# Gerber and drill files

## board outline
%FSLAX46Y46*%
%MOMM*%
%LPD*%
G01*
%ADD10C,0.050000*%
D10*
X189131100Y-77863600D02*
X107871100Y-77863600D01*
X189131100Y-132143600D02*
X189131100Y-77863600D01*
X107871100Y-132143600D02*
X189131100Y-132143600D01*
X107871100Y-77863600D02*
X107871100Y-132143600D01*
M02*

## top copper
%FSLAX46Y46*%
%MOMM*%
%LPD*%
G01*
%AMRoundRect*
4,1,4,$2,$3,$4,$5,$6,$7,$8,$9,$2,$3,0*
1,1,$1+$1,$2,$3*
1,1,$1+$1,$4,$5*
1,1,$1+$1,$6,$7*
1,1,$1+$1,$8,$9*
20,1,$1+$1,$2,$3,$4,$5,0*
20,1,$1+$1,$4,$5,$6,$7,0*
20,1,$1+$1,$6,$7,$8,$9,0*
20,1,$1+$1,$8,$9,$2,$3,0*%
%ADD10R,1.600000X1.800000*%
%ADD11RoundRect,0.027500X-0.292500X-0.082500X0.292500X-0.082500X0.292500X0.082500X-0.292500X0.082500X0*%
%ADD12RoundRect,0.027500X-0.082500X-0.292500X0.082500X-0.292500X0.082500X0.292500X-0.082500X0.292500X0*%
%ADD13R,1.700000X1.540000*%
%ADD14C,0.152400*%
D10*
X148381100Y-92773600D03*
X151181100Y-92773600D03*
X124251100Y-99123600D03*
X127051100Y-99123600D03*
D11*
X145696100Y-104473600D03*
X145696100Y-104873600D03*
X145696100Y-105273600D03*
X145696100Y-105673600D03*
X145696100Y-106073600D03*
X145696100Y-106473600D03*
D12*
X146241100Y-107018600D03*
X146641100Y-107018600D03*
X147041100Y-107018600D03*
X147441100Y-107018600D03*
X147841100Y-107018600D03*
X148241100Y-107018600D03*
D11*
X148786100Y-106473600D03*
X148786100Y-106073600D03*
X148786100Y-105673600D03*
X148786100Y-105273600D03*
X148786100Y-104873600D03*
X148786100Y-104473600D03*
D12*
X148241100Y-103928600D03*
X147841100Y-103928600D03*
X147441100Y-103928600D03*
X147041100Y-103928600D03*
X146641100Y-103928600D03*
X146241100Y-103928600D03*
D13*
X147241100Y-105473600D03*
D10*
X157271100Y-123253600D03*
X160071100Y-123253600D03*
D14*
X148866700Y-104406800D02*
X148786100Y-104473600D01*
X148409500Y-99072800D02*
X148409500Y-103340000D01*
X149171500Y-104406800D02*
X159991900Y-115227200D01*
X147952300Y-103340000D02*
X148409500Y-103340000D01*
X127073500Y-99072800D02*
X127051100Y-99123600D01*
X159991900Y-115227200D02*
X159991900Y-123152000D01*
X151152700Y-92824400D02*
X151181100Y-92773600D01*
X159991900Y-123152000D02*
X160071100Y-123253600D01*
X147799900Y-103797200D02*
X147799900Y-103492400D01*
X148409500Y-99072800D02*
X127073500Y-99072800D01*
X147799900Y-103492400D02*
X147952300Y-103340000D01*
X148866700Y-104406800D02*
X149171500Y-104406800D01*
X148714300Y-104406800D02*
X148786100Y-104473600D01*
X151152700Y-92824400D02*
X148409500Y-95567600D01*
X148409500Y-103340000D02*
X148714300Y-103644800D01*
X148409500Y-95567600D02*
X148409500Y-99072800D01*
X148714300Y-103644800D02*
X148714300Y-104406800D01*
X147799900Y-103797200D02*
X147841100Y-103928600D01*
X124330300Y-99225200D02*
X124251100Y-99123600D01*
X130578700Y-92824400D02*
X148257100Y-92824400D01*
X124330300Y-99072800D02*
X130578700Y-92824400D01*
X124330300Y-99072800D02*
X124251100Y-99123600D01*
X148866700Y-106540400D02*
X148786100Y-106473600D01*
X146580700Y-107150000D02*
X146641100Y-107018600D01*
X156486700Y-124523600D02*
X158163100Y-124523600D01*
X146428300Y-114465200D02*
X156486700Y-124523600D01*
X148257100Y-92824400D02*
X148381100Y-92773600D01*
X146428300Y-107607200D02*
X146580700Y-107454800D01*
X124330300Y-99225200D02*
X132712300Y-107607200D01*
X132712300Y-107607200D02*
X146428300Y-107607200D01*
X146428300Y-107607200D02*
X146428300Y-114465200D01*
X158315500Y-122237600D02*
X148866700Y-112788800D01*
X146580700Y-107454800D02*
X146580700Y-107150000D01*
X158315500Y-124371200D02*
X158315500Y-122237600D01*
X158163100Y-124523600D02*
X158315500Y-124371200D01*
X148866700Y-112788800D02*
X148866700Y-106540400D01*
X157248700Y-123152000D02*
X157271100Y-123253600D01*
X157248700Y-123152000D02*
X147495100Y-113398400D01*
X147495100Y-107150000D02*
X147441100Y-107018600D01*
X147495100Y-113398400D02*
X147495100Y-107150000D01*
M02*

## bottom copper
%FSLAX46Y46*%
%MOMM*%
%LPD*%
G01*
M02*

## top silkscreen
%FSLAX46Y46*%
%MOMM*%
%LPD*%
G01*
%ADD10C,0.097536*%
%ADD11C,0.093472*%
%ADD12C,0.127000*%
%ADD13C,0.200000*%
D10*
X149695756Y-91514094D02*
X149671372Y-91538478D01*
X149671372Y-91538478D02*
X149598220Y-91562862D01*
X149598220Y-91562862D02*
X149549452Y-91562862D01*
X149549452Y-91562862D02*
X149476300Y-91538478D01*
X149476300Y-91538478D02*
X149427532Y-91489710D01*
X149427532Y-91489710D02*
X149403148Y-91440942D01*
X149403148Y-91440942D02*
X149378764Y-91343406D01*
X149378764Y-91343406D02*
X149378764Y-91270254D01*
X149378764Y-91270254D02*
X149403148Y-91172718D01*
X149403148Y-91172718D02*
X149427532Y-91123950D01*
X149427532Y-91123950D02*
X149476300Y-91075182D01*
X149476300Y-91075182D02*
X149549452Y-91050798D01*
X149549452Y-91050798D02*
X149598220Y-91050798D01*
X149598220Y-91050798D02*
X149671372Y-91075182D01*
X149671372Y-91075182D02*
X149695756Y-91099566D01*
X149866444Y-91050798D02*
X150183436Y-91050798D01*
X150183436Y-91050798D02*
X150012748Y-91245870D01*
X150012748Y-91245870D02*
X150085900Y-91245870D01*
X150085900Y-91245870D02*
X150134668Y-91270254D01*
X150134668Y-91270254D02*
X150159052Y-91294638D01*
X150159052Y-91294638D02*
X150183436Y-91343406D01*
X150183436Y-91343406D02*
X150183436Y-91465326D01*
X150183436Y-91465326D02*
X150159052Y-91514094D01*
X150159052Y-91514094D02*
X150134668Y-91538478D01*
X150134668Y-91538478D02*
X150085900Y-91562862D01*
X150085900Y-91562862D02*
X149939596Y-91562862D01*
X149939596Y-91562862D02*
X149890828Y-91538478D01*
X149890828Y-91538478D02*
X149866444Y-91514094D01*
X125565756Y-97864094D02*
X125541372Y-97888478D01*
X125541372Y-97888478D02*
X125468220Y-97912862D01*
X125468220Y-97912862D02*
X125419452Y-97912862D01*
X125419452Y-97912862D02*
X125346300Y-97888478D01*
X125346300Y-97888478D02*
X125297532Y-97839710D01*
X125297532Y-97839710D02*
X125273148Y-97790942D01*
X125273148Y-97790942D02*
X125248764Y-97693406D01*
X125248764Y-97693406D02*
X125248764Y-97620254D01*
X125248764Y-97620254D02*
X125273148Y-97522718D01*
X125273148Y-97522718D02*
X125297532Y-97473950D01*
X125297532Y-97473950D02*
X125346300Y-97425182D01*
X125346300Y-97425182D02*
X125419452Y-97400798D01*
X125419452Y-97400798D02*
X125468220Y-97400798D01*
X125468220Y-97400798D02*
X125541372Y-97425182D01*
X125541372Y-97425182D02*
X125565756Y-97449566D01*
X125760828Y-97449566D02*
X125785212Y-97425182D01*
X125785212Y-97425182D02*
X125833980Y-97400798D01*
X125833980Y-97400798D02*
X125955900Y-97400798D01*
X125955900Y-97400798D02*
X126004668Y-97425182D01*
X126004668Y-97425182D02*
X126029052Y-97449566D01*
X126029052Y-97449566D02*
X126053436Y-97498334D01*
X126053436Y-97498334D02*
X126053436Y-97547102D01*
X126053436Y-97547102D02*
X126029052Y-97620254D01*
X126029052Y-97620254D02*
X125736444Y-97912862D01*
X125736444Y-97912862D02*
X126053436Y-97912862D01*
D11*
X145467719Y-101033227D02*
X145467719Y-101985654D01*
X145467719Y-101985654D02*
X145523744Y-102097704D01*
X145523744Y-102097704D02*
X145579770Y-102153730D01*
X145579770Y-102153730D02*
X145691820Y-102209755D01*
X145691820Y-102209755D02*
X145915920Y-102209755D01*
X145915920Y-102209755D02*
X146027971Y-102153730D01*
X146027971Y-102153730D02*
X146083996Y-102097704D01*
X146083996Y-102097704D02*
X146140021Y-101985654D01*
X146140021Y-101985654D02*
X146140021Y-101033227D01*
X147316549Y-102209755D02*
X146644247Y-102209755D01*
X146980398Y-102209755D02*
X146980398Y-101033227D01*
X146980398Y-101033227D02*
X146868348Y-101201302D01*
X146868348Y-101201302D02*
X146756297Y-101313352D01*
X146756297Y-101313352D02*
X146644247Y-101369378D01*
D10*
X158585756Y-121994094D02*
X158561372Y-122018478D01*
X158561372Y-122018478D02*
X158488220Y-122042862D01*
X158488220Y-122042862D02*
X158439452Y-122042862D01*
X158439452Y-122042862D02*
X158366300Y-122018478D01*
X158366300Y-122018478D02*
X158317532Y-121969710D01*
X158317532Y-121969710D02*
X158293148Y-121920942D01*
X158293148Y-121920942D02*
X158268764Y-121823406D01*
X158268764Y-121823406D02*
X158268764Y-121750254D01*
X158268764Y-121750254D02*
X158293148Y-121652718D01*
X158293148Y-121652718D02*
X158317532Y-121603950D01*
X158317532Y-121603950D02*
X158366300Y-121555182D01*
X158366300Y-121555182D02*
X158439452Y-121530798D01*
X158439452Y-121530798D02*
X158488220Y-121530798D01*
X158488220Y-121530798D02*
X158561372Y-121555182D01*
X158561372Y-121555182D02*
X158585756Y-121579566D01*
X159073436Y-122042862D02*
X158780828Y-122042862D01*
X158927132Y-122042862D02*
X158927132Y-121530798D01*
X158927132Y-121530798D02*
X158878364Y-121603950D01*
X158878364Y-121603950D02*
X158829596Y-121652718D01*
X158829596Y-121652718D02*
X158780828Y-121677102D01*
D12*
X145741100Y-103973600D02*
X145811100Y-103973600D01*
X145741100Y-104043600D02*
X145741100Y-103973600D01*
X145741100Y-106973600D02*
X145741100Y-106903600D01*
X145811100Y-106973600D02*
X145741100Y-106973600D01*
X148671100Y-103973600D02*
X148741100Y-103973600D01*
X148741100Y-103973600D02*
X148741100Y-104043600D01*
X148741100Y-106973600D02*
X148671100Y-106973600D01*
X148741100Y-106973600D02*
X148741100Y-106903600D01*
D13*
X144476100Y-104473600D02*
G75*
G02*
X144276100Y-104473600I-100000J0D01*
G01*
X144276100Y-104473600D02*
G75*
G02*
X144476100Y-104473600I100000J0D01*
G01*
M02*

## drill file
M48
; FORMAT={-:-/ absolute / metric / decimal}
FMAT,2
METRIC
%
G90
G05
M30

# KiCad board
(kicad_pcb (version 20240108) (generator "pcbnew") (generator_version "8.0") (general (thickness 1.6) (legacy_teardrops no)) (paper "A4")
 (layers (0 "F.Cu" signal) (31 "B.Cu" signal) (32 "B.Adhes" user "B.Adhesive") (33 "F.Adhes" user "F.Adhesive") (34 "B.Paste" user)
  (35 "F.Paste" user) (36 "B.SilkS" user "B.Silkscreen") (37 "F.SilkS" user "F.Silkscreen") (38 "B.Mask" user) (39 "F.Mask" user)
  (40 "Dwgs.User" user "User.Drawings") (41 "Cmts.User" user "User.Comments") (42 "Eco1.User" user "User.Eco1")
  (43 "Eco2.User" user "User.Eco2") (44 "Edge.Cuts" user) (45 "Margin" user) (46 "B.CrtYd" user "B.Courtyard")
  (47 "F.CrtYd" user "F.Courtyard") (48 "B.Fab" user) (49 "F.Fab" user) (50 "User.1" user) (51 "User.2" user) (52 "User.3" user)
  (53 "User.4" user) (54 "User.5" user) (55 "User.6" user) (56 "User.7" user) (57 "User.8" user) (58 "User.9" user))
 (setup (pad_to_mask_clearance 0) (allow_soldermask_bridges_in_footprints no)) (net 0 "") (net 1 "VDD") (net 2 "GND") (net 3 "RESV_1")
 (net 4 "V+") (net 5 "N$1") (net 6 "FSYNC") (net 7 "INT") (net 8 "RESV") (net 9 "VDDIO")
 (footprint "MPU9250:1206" (layer "F.Cu") (at 149.7811 92.7736)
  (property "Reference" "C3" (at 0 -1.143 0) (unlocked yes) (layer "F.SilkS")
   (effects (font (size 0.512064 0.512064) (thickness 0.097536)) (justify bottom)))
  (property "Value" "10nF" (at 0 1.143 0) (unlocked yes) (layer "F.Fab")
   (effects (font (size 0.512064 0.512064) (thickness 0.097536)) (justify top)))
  (pad "1" smd rect (at -1.4 0) (size 1.6 1.8) (layers "F.Cu" "F.Paste" "F.Mask") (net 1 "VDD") (solder_mask_margin 0.1016)
   (thermal_bridge_angle 0))
  (pad "2" smd rect (at 1.4 0) (size 1.6 1.8) (layers "F.Cu" "F.Paste" "F.Mask") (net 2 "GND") (solder_mask_margin 0.1016)
   (thermal_bridge_angle 0)))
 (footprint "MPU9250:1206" (layer "F.Cu") (at 125.6511 99.1236)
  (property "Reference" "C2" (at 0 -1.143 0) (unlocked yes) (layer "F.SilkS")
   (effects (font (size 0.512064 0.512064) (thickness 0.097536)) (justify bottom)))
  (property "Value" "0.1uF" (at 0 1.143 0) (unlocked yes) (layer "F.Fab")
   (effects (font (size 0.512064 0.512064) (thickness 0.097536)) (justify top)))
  (pad "1" smd rect (at -1.4 0) (size 1.6 1.8) (layers "F.Cu" "F.Paste" "F.Mask") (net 1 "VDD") (solder_mask_margin 0.1016)
   (thermal_bridge_angle 0))
  (pad "2" smd rect (at 1.4 0) (size 1.6 1.8) (layers "F.Cu" "F.Paste" "F.Mask") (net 2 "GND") (solder_mask_margin 0.1016)
   (thermal_bridge_angle 0)))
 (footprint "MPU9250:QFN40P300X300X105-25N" (layer "F.Cu") (at 147.2411 105.4736)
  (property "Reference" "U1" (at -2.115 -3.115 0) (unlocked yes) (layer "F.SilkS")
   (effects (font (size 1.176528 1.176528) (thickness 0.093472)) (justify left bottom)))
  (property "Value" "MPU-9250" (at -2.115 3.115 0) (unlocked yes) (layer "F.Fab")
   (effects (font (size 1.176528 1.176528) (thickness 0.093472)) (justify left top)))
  (fp_line (start -1.5 -1.5) (end -1.43 -1.5) (stroke (width 0.127) (type solid)) (layer "F.SilkS"))
  (fp_line (start -1.5 -1.43) (end -1.5 -1.5) (stroke (width 0.127) (type solid)) (layer "F.SilkS"))
  (fp_line (start -1.5 1.5) (end -1.5 1.43) (stroke (width 0.127) (type solid)) (layer "F.SilkS"))
  (fp_line (start -1.43 1.5) (end -1.5 1.5) (stroke (width 0.127) (type solid)) (layer "F.SilkS"))
  (fp_line (start 1.43 -1.5) (end 1.5 -1.5) (stroke (width 0.127) (type solid)) (layer "F.SilkS"))
  (fp_line (start 1.5 -1.5) (end 1.5 -1.43) (stroke (width 0.127) (type solid)) (layer "F.SilkS"))
  (fp_line (start 1.5 1.5) (end 1.43 1.5) (stroke (width 0.127) (type solid)) (layer "F.SilkS"))
  (fp_line (start 1.5 1.5) (end 1.5 1.43) (stroke (width 0.127) (type solid)) (layer "F.SilkS"))
  (fp_circle (center -2.865 -1) (end -2.765 -1) (stroke (width 0.2) (type solid)) (fill none) (layer "F.SilkS"))
  (pad "1" smd roundrect (at -1.545 -1) (size 0.64 0.22) (layers "F.Cu" "F.Paste" "F.Mask") (roundrect_rratio 0.125) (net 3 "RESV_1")
   (solder_mask_margin 0.1016) (thermal_bridge_angle 0))
  (pad "2" smd roundrect (at -1.545 -0.6) (size 0.64 0.22) (layers "F.Cu" "F.Paste" "F.Mask") (roundrect_rratio 0.125)
   (solder_mask_margin 0.1016) (thermal_bridge_angle 0))
  (pad "3" smd roundrect (at -1.545 -0.2) (size 0.64 0.22) (layers "F.Cu" "F.Paste" "F.Mask") (roundrect_rratio 0.125)
   (solder_mask_margin 0.1016) (thermal_bridge_angle 0))
  (pad "4" smd roundrect (at -1.545 0.2) (size 0.64 0.22) (layers "F.Cu" "F.Paste" "F.Mask") (roundrect_rratio 0.125)
   (solder_mask_margin 0.1016) (thermal_bridge_angle 0))
  (pad "5" smd roundrect (at -1.545 0.6) (size 0.64 0.22) (layers "F.Cu" "F.Paste" "F.Mask") (roundrect_rratio 0.125)
   (solder_mask_margin 0.1016) (thermal_bridge_angle 0))
  (pad "6" smd roundrect (at -1.545 1) (size 0.64 0.22) (layers "F.Cu" "F.Paste" "F.Mask") (roundrect_rratio 0.125)
   (solder_mask_margin 0.1016) (thermal_bridge_angle 0))
  (pad "7" smd roundrect (at -1 1.545) (size 0.22 0.64) (layers "F.Cu" "F.Paste" "F.Mask") (roundrect_rratio 0.125)
   (solder_mask_margin 0.1016) (thermal_bridge_angle 0))
  (pad "8" smd roundrect (at -0.6 1.545) (size 0.22 0.64) (layers "F.Cu" "F.Paste" "F.Mask") (roundrect_rratio 0.125) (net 1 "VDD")
   (solder_mask_margin 0.1016) (thermal_bridge_angle 0))
  (pad "9" smd roundrect (at -0.2 1.545) (size 0.22 0.64) (layers "F.Cu" "F.Paste" "F.Mask") (roundrect_rratio 0.125) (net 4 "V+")
   (solder_mask_margin 0.1016) (thermal_bridge_angle 0))
  (pad "10" smd roundrect (at 0.2 1.545) (size 0.22 0.64) (layers "F.Cu" "F.Paste" "F.Mask") (roundrect_rratio 0.125) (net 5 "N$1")
   (solder_mask_margin 0.1016) (thermal_bridge_angle 0))
  (pad "11" smd roundrect (at 0.6 1.545) (size 0.22 0.64) (layers "F.Cu" "F.Paste" "F.Mask") (roundrect_rratio 0.125) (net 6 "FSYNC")
   (solder_mask_margin 0.1016) (thermal_bridge_angle 0))
  (pad "12" smd roundrect (at 1 1.545) (size 0.22 0.64) (layers "F.Cu" "F.Paste" "F.Mask") (roundrect_rratio 0.125) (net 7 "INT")
   (solder_mask_margin 0.1016) (thermal_bridge_angle 0))
  (pad "13" smd roundrect (at 1.545 1) (size 0.64 0.22) (layers "F.Cu" "F.Paste" "F.Mask") (roundrect_rratio 0.125) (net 1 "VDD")
   (solder_mask_margin 0.1016) (thermal_bridge_angle 0))
  (pad "14" smd roundrect (at 1.545 0.6) (size 0.64 0.22) (layers "F.Cu" "F.Paste" "F.Mask") (roundrect_rratio 0.125)
   (solder_mask_margin 0.1016) (thermal_bridge_angle 0))
  (pad "15" smd roundrect (at 1.545 0.2) (size 0.64 0.22) (layers "F.Cu" "F.Paste" "F.Mask") (roundrect_rratio 0.125)
   (solder_mask_margin 0.1016) (thermal_bridge_angle 0))
  (pad "16" smd roundrect (at 1.545 -0.2) (size 0.64 0.22) (layers "F.Cu" "F.Paste" "F.Mask") (roundrect_rratio 0.125)
   (solder_mask_margin 0.1016) (thermal_bridge_angle 0))
  (pad "17" smd roundrect (at 1.545 -0.6) (size 0.64 0.22) (layers "F.Cu" "F.Paste" "F.Mask") (roundrect_rratio 0.125)
   (solder_mask_margin 0.1016) (thermal_bridge_angle 0))
  (pad "18" smd roundrect (at 1.545 -1) (size 0.64 0.22) (layers "F.Cu" "F.Paste" "F.Mask") (roundrect_rratio 0.125) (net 2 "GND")
   (solder_mask_margin 0.1016) (thermal_bridge_angle 0))
  (pad "19" smd roundrect (at 1 -1.545) (size 0.22 0.64) (layers "F.Cu" "F.Paste" "F.Mask") (roundrect_rratio 0.125) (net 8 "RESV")
   (solder_mask_margin 0.1016) (thermal_bridge_angle 0))
  (pad "20" smd roundrect (at 0.6 -1.545) (size 0.22 0.64) (layers "F.Cu" "F.Paste" "F.Mask") (roundrect_rratio 0.125) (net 2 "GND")
   (solder_mask_margin 0.1016) (thermal_bridge_angle 0))
  (pad "21" smd roundrect (at 0.2 -1.545) (size 0.22 0.64) (layers "F.Cu" "F.Paste" "F.Mask") (roundrect_rratio 0.125)
   (solder_mask_margin 0.1016) (thermal_bridge_angle 0))
  (pad "22" smd roundrect (at -0.2 -1.545) (size 0.22 0.64) (layers "F.Cu" "F.Paste" "F.Mask") (roundrect_rratio 0.125) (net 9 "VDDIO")
   (solder_mask_margin 0.1016) (thermal_bridge_angle 0))
  (pad "23" smd roundrect (at -0.6 -1.545) (size 0.22 0.64) (layers "F.Cu" "F.Paste" "F.Mask") (roundrect_rratio 0.125)
   (solder_mask_margin 0.1016) (thermal_bridge_angle 0))
  (pad "24" smd roundrect (at -1 -1.545) (size 0.22 0.64) (layers "F.Cu" "F.Paste" "F.Mask") (roundrect_rratio 0.125)
   (solder_mask_margin 0.1016) (thermal_bridge_angle 0))
  (pad "25" smd rect (at 0 0) (size 1.7 1.54) (layers "F.Cu" "F.Mask") (solder_mask_margin 0.1016) (thermal_bridge_angle 0)))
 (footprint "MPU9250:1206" (layer "F.Cu") (at 158.6711 123.2536)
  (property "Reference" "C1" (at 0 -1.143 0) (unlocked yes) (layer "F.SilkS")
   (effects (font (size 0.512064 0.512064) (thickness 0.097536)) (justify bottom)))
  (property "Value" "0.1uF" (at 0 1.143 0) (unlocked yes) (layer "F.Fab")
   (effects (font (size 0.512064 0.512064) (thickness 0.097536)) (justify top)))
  (pad "1" smd rect (at -1.4 0) (size 1.6 1.8) (layers "F.Cu" "F.Paste" "F.Mask") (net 5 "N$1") (solder_mask_margin 0.1016)
   (thermal_bridge_angle 0))
  (pad "2" smd rect (at 1.4 0) (size 1.6 1.8) (layers "F.Cu" "F.Paste" "F.Mask") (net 2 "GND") (solder_mask_margin 0.1016)
   (thermal_bridge_angle 0)))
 (gr_line (start 189.1311 77.8636) (end 107.8711 77.8636) (stroke (width 0.05) (type solid)) (layer "Edge.Cuts"))
 (gr_line (start 189.1311 132.1436) (end 189.1311 77.8636) (stroke (width 0.05) (type solid)) (layer "Edge.Cuts"))
 (gr_line (start 107.8711 132.1436) (end 189.1311 132.1436) (stroke (width 0.05) (type solid)) (layer "Edge.Cuts"))
 (gr_line (start 107.8711 77.8636) (end 107.8711 132.1436) (stroke (width 0.05) (type solid)) (layer "Edge.Cuts"))
 (segment (start 148.8667 104.4068) (end 148.7861 104.4736) (width 0.1524) (layer "F.Cu") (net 2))
 (segment (start 148.4095 99.0728) (end 148.4095 103.34) (width 0.1524) (layer "F.Cu") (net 2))
 (segment (start 149.1715 104.4068) (end 159.9919 115.2272) (width 0.1524) (layer "F.Cu") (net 2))
 (segment (start 147.9523 103.34) (end 148.4095 103.34) (width 0.1524) (layer "F.Cu") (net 2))
 (segment (start 127.0735 99.0728) (end 127.0511 99.1236) (width 0.1524) (layer "F.Cu") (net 2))
 (segment (start 159.9919 115.2272) (end 159.9919 123.152) (width 0.1524) (layer "F.Cu") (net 2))
 (segment (start 151.1527 92.8244) (end 151.1811 92.7736) (width 0.1524) (layer "F.Cu") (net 2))
 (segment (start 159.9919 123.152) (end 160.0711 123.2536) (width 0.1524) (layer "F.Cu") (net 2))
 (segment (start 147.7999 103.7972) (end 147.7999 103.4924) (width 0.1524) (layer "F.Cu") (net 2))
 (segment (start 148.4095 99.0728) (end 127.0735 99.0728) (width 0.1524) (layer "F.Cu") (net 2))
 (segment (start 147.7999 103.4924) (end 147.9523 103.34) (width 0.1524) (layer "F.Cu") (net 2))
 (segment (start 148.8667 104.4068) (end 149.1715 104.4068) (width 0.1524) (layer "F.Cu") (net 2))
 (segment (start 148.7143 104.4068) (end 148.7861 104.4736) (width 0.1524) (layer "F.Cu") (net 2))
 (segment (start 151.1527 92.8244) (end 148.4095 95.5676) (width 0.1524) (layer "F.Cu") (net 2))
 (segment (start 148.4095 103.34) (end 148.7143 103.6448) (width 0.1524) (layer "F.Cu") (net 2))
 (segment (start 148.4095 95.5676) (end 148.4095 99.0728) (width 0.1524) (layer "F.Cu") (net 2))
 (segment (start 148.7143 103.6448) (end 148.7143 104.4068) (width 0.1524) (layer "F.Cu") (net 2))
 (segment (start 147.7999 103.7972) (end 147.8411 103.9286) (width 0.1524) (layer "F.Cu") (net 2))
 (segment (start 124.3303 99.2252) (end 124.2511 99.1236) (width 0.1524) (layer "F.Cu") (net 1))
 (segment (start 130.5787 92.8244) (end 148.2571 92.8244) (width 0.1524) (layer "F.Cu") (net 1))
 (segment (start 124.3303 99.0728) (end 130.5787 92.8244) (width 0.1524) (layer "F.Cu") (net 1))
 (segment (start 124.3303 99.0728) (end 124.2511 99.1236) (width 0.1524) (layer "F.Cu") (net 1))
 (segment (start 148.8667 106.5404) (end 148.7861 106.4736) (width 0.1524) (layer "F.Cu") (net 1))
 (segment (start 146.5807 107.15) (end 146.6411 107.0186) (width 0.1524) (layer "F.Cu") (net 1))
 (segment (start 156.4867 124.5236) (end 158.1631 124.5236) (width 0.1524) (layer "F.Cu") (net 1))
 (segment (start 146.4283 114.4652) (end 156.4867 124.5236) (width 0.1524) (layer "F.Cu") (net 1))
 (segment (start 148.2571 92.8244) (end 148.3811 92.7736) (width 0.1524) (layer "F.Cu") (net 1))
 (segment (start 146.4283 107.6072) (end 146.5807 107.4548) (width 0.1524) (layer "F.Cu") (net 1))
 (segment (start 124.3303 99.2252) (end 132.7123 107.6072) (width 0.1524) (layer "F.Cu") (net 1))
 (segment (start 132.7123 107.6072) (end 146.4283 107.6072) (width 0.1524) (layer "F.Cu") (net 1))
 (segment (start 146.4283 107.6072) (end 146.4283 114.4652) (width 0.1524) (layer "F.Cu") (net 1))
 (segment (start 158.3155 122.2376) (end 148.8667 112.7888) (width 0.1524) (layer "F.Cu") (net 1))
 (segment (start 146.5807 107.4548) (end 146.5807 107.15) (width 0.1524) (layer "F.Cu") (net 1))
 (segment (start 158.3155 124.3712) (end 158.3155 122.2376) (width 0.1524) (layer "F.Cu") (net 1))
 (segment (start 158.1631 124.5236) (end 158.3155 124.3712) (width 0.1524) (layer "F.Cu") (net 1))
 (segment (start 148.8667 112.7888) (end 148.8667 106.5404) (width 0.1524) (layer "F.Cu") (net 1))
 (segment (start 157.2487 123.152) (end 157.2711 123.2536) (width 0.1524) (layer "F.Cu") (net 5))
 (segment (start 157.2487 123.152) (end 147.4951 113.3984) (width 0.1524) (layer "F.Cu") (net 5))
 (segment (start 147.4951 107.15) (end 147.4411 107.0186) (width 0.1524) (layer "F.Cu") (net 5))
 (segment (start 147.4951 113.3984) (end 147.4951 107.15) (width 0.1524) (layer "F.Cu") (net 5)))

